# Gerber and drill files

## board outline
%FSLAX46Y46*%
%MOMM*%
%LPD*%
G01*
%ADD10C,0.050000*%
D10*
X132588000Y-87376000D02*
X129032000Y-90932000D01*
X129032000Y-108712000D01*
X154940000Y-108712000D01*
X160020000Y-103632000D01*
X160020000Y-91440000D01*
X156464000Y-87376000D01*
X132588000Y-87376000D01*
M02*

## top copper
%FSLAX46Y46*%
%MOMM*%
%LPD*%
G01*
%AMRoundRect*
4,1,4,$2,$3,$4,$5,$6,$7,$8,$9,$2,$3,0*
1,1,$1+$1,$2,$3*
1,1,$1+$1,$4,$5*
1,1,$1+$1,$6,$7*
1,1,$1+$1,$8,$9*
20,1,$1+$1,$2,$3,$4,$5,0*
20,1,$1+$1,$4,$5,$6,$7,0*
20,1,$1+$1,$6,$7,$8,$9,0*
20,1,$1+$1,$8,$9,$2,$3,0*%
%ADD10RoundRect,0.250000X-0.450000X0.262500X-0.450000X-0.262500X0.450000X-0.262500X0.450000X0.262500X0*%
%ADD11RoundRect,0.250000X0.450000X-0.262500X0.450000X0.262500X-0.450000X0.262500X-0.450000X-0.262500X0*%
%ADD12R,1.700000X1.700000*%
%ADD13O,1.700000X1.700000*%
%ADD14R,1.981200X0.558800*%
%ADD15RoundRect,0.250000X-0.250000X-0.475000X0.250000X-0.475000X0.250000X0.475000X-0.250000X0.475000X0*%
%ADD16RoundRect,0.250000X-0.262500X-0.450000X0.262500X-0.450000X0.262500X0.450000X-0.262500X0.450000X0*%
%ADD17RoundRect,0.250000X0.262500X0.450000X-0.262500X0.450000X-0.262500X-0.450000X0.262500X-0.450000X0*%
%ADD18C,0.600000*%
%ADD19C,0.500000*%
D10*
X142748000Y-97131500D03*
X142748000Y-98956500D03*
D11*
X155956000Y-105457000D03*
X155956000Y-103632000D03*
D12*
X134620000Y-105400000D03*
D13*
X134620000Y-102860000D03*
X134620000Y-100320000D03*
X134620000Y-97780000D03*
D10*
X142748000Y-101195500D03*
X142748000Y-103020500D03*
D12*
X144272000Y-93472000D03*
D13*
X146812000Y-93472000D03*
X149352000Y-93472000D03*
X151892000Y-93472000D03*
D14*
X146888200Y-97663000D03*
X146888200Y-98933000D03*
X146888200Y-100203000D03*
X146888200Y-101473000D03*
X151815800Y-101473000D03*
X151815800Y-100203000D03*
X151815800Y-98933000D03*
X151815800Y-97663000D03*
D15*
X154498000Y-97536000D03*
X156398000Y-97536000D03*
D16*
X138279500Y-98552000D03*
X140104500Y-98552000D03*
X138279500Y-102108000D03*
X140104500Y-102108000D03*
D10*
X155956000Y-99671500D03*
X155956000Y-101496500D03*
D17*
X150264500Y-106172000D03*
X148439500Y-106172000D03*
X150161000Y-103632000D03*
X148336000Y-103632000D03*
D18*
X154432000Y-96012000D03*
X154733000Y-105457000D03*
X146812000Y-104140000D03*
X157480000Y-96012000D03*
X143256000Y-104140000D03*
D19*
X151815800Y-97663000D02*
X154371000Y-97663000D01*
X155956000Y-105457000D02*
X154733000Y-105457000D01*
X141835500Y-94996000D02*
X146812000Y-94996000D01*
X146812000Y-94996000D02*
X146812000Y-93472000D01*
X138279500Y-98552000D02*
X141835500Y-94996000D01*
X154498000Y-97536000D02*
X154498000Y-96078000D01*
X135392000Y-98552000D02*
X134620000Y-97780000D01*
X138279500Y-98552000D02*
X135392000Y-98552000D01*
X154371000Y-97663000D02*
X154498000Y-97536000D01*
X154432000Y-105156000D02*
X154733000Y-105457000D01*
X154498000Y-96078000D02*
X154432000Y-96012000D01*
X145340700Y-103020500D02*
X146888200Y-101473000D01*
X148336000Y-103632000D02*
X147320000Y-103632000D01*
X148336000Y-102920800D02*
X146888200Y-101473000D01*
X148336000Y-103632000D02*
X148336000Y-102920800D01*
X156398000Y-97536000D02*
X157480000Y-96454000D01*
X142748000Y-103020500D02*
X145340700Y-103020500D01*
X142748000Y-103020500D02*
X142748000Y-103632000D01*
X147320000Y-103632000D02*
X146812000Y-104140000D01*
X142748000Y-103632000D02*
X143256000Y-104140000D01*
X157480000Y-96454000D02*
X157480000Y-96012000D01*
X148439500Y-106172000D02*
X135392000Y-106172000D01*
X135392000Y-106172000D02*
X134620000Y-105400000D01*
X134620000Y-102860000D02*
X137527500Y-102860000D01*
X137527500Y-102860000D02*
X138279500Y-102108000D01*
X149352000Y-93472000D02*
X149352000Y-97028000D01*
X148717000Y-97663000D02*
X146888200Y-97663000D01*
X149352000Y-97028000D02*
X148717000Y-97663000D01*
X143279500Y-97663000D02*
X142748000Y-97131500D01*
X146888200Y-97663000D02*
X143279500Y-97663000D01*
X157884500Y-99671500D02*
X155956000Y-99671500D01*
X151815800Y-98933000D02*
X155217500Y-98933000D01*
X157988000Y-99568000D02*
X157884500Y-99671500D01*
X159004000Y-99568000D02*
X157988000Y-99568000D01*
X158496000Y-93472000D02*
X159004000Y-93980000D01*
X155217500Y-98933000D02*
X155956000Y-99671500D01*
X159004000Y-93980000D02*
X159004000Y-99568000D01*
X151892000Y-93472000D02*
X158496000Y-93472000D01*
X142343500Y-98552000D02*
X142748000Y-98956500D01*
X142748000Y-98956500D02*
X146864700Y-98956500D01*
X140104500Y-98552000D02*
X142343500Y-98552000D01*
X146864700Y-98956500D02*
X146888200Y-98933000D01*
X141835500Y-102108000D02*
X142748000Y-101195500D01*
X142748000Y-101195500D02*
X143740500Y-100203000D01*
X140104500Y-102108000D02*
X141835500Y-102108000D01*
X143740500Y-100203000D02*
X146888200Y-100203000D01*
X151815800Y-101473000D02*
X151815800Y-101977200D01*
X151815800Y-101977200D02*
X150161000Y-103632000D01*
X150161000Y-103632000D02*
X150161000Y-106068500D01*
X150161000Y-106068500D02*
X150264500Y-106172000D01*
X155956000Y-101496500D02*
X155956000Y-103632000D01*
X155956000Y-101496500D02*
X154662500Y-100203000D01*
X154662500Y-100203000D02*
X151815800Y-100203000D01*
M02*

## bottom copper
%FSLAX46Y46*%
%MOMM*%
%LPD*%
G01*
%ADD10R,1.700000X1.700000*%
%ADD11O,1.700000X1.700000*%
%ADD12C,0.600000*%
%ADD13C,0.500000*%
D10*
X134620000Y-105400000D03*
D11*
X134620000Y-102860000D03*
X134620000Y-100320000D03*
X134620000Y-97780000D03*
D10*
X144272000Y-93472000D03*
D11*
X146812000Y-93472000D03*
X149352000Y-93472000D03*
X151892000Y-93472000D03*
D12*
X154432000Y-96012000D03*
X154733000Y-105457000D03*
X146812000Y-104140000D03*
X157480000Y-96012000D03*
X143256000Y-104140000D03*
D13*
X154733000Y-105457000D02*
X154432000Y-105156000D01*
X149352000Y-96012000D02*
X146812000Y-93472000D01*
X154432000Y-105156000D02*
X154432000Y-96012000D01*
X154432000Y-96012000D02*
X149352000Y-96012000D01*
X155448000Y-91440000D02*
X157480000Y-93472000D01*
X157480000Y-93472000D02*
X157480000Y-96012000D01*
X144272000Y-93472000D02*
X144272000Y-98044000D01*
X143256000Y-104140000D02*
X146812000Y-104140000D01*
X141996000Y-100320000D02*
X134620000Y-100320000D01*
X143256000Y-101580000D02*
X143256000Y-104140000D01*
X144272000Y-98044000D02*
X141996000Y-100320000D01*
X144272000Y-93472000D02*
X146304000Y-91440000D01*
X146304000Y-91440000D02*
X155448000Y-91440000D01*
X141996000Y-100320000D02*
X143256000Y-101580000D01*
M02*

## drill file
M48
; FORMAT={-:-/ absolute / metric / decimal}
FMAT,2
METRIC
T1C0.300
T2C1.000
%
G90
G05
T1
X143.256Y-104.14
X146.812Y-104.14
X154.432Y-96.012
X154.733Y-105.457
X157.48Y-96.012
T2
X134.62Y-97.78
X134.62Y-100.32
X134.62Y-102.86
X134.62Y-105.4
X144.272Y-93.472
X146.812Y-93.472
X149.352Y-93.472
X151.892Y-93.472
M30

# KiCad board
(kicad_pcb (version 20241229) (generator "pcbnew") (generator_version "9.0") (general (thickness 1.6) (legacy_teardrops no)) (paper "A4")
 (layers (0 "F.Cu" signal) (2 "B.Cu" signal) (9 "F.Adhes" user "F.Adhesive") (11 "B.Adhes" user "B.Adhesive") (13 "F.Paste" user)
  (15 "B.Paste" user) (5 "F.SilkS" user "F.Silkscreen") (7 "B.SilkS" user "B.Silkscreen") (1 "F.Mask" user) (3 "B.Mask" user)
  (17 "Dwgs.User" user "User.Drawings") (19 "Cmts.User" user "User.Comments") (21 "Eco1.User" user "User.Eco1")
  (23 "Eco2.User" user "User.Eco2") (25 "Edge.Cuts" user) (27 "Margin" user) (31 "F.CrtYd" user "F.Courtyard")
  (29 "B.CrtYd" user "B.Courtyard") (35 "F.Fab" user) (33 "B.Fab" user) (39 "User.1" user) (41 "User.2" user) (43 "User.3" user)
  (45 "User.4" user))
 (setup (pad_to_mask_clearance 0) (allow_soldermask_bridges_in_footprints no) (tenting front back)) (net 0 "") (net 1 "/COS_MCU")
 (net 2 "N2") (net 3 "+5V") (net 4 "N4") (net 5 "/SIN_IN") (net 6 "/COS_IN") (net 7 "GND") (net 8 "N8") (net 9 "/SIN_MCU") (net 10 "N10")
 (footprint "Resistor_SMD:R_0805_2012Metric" (layer "F.Cu") (at 142.748 98.044 -90)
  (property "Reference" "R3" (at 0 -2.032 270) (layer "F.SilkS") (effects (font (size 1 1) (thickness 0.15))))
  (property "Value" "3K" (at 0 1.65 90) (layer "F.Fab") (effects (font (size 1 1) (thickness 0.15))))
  (pad "1" smd roundrect (at -0.9125 0 270) (size 1.025 1.4) (layers "F.Cu" "F.Mask" "F.Paste") (roundrect_rratio 0.243902)
   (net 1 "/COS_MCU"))
  (pad "2" smd roundrect (at 0.9125 0 270) (size 1.025 1.4) (layers "F.Cu" "F.Mask" "F.Paste") (roundrect_rratio 0.243902) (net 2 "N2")))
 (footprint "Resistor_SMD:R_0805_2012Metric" (layer "F.Cu") (at 155.956 104.5445 90)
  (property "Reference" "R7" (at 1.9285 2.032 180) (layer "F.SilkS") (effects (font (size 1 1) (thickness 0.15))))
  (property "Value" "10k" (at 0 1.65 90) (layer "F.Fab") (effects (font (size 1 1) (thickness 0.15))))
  (pad "1" smd roundrect (at -0.9125 0 90) (size 1.025 1.4) (layers "F.Cu" "F.Mask" "F.Paste") (roundrect_rratio 0.243902) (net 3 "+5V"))
  (pad "2" smd roundrect (at 0.9125 0 90) (size 1.025 1.4) (layers "F.Cu" "F.Mask" "F.Paste") (roundrect_rratio 0.243902) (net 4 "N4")))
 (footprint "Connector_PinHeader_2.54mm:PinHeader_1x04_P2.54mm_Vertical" (layer "F.Cu") (at 134.62 105.4 180)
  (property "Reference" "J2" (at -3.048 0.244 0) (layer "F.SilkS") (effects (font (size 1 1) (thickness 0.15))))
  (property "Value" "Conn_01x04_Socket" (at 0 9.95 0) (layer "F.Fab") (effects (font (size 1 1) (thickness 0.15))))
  (pad "1" thru_hole rect (at 0 0 180) (size 1.7 1.7) (drill 1) (layers "*.Cu" "*.Mask") (remove_unused_layers no) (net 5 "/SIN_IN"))
  (pad "2" thru_hole oval (at 0 2.54 180) (size 1.7 1.7) (drill 1) (layers "*.Cu" "*.Mask") (remove_unused_layers no) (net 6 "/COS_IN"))
  (pad "3" thru_hole oval (at 0 5.08 180) (size 1.7 1.7) (drill 1) (layers "*.Cu" "*.Mask") (remove_unused_layers no) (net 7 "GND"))
  (pad "4" thru_hole oval (at 0 7.62 180) (size 1.7 1.7) (drill 1) (layers "*.Cu" "*.Mask") (remove_unused_layers no) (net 3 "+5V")))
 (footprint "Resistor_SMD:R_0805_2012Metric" (layer "F.Cu") (at 142.748 102.108 -90)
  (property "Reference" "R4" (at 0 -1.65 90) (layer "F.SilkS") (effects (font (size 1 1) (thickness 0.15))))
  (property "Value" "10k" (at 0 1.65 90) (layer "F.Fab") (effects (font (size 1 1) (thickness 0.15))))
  (pad "1" smd roundrect (at -0.9125 0 270) (size 1.025 1.4) (layers "F.Cu" "F.Mask" "F.Paste") (roundrect_rratio 0.243902) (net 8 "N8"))
  (pad "2" smd roundrect (at 0.9125 0 270) (size 1.025 1.4) (layers "F.Cu" "F.Mask" "F.Paste") (roundrect_rratio 0.243902) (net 7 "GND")))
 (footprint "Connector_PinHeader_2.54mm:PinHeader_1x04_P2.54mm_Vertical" (layer "F.Cu") (at 144.272 93.472 90)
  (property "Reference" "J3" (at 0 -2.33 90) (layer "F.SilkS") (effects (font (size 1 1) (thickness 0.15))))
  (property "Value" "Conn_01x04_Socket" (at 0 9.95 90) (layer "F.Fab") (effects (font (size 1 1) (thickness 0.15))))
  (pad "1" thru_hole rect (at 0 0 90) (size 1.7 1.7) (drill 1) (layers "*.Cu" "*.Mask") (remove_unused_layers no) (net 7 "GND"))
  (pad "2" thru_hole oval (at 0 2.54 90) (size 1.7 1.7) (drill 1) (layers "*.Cu" "*.Mask") (remove_unused_layers no) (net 3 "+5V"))
  (pad "3" thru_hole oval (at 0 5.08 90) (size 1.7 1.7) (drill 1) (layers "*.Cu" "*.Mask") (remove_unused_layers no) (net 1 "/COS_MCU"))
  (pad "4" thru_hole oval (at 0 7.62 90) (size 1.7 1.7) (drill 1) (layers "*.Cu" "*.Mask") (remove_unused_layers no) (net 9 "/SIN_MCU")))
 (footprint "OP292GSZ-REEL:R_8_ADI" (layer "F.Cu") (at 149.352 99.568)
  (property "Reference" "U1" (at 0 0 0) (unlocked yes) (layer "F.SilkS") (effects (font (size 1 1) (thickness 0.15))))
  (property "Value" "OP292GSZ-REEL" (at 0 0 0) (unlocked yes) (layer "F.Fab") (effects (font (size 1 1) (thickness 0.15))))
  (pad "1" smd rect (at -2.4638 -1.905) (size 1.9812 0.5588) (layers "F.Cu" "F.Mask" "F.Paste") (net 1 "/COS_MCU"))
  (pad "2" smd rect (at -2.4638 -0.635) (size 1.9812 0.5588) (layers "F.Cu" "F.Mask" "F.Paste") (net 2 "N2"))
  (pad "3" smd rect (at -2.4638 0.635) (size 1.9812 0.5588) (layers "F.Cu" "F.Mask" "F.Paste") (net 8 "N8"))
  (pad "4" smd rect (at -2.4638 1.905) (size 1.9812 0.5588) (layers "F.Cu" "F.Mask" "F.Paste") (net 7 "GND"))
  (pad "5" smd rect (at 2.4638 1.905) (size 1.9812 0.5588) (layers "F.Cu" "F.Mask" "F.Paste") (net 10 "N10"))
  (pad "6" smd rect (at 2.4638 0.635) (size 1.9812 0.5588) (layers "F.Cu" "F.Mask" "F.Paste") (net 4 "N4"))
  (pad "7" smd rect (at 2.4638 -0.635) (size 1.9812 0.5588) (layers "F.Cu" "F.Mask" "F.Paste") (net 9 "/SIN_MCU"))
  (pad "8" smd rect (at 2.4638 -1.905) (size 1.9812 0.5588) (layers "F.Cu" "F.Mask" "F.Paste") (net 3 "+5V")))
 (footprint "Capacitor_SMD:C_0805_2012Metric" (layer "F.Cu") (at 155.448 97.536)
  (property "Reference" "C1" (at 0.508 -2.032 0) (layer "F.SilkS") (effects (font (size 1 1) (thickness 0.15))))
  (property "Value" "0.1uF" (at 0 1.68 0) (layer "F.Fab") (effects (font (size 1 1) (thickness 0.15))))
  (pad "1" smd roundrect (at -0.95 0) (size 1 1.45) (layers "F.Cu" "F.Mask" "F.Paste") (roundrect_rratio 0.25) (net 3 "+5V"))
  (pad "2" smd roundrect (at 0.95 0) (size 1 1.45) (layers "F.Cu" "F.Mask" "F.Paste") (roundrect_rratio 0.25) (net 7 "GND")))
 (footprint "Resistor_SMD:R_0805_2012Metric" (layer "F.Cu") (at 139.192 98.552)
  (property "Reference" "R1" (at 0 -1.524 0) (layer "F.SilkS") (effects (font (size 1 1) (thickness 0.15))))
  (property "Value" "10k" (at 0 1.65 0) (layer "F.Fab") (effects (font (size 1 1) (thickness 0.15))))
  (pad "1" smd roundrect (at -0.9125 0) (size 1.025 1.4) (layers "F.Cu" "F.Mask" "F.Paste") (roundrect_rratio 0.243902) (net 3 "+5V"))
  (pad "2" smd roundrect (at 0.9125 0) (size 1.025 1.4) (layers "F.Cu" "F.Mask" "F.Paste") (roundrect_rratio 0.243902) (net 2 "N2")))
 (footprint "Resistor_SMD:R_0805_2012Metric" (layer "F.Cu") (at 139.192 102.108)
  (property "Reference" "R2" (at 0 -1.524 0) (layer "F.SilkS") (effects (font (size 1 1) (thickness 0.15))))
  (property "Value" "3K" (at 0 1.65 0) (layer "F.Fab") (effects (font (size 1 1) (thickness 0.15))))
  (pad "1" smd roundrect (at -0.9125 0) (size 1.025 1.4) (layers "F.Cu" "F.Mask" "F.Paste") (roundrect_rratio 0.243902) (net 6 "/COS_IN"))
  (pad "2" smd roundrect (at 0.9125 0) (size 1.025 1.4) (layers "F.Cu" "F.Mask" "F.Paste") (roundrect_rratio 0.243902) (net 8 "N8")))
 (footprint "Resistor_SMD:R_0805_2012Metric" (layer "F.Cu") (at 155.956 100.584 -90)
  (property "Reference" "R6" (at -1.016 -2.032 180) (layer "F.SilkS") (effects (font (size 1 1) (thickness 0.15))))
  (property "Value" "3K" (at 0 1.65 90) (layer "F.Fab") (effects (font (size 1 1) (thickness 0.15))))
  (pad "1" smd roundrect (at -0.9125 0 270) (size 1.025 1.4) (layers "F.Cu" "F.Mask" "F.Paste") (roundrect_rratio 0.243902)
   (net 9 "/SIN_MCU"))
  (pad "2" smd roundrect (at 0.9125 0 270) (size 1.025 1.4) (layers "F.Cu" "F.Mask" "F.Paste") (roundrect_rratio 0.243902) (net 4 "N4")))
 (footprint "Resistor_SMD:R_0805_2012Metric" (layer "F.Cu") (at 149.352 106.172 180)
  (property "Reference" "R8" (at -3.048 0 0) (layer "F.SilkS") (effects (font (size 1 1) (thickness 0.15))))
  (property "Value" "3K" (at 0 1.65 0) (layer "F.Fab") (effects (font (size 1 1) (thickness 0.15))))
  (pad "1" smd roundrect (at -0.9125 0 180) (size 1.025 1.4) (layers "F.Cu" "F.Mask" "F.Paste") (roundrect_rratio 0.243902) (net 10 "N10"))
  (pad "2" smd roundrect (at 0.9125 0 180) (size 1.025 1.4) (layers "F.Cu" "F.Mask" "F.Paste") (roundrect_rratio 0.243902) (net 5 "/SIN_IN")))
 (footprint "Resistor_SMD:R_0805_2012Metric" (layer "F.Cu") (at 149.2485 103.632 180)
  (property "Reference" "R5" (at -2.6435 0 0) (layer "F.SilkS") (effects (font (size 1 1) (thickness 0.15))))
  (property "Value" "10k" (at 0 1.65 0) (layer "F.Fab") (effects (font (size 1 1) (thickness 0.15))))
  (pad "1" smd roundrect (at -0.9125 0 180) (size 1.025 1.4) (layers "F.Cu" "F.Mask" "F.Paste") (roundrect_rratio 0.243902) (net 10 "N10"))
  (pad "2" smd roundrect (at 0.9125 0 180) (size 1.025 1.4) (layers "F.Cu" "F.Mask" "F.Paste") (roundrect_rratio 0.243902) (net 7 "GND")))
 (gr_poly
  (pts (xy 132.588 87.376) (xy 129.032 90.932) (xy 129.032 108.712) (xy 154.94 108.712) (xy 160.02 103.632) (xy 160.02 91.44)
   (xy 156.464 87.376))
  (stroke (width 0.05) (type solid)) (fill no) (layer "Edge.Cuts"))
 (segment (start 151.8158 97.663) (end 154.371 97.663) (width 0.5) (layer "F.Cu") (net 3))
 (segment (start 155.956 105.457) (end 154.733 105.457) (width 0.5) (layer "F.Cu") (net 3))
 (segment (start 141.8355 94.996) (end 146.812 94.996) (width 0.5) (layer "F.Cu") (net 3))
 (segment (start 146.812 94.996) (end 146.812 93.472) (width 0.5) (layer "F.Cu") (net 3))
 (segment (start 138.2795 98.552) (end 141.8355 94.996) (width 0.5) (layer "F.Cu") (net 3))
 (segment (start 154.498 97.536) (end 154.498 96.078) (width 0.5) (layer "F.Cu") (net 3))
 (segment (start 135.392 98.552) (end 134.62 97.78) (width 0.5) (layer "F.Cu") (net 3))
 (segment (start 138.2795 98.552) (end 135.392 98.552) (width 0.5) (layer "F.Cu") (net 3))
 (segment (start 154.371 97.663) (end 154.498 97.536) (width 0.5) (layer "F.Cu") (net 3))
 (segment (start 154.432 105.156) (end 154.733 105.457) (width 0.5) (layer "F.Cu") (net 3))
 (segment (start 154.498 96.078) (end 154.432 96.012) (width 0.5) (layer "F.Cu") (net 3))
 (via (at 154.432 96.012) (size 0.6) (drill 0.3) (layers "F.Cu" "B.Cu") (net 3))
 (via (at 154.733 105.457) (size 0.6) (drill 0.3) (layers "F.Cu" "B.Cu") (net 3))
 (segment (start 154.733 105.457) (end 154.432 105.156) (width 0.5) (layer "B.Cu") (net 3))
 (segment (start 149.352 96.012) (end 146.812 93.472) (width 0.5) (layer "B.Cu") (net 3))
 (segment (start 154.432 105.156) (end 154.432 96.012) (width 0.5) (layer "B.Cu") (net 3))
 (segment (start 154.432 96.012) (end 149.352 96.012) (width 0.5) (layer "B.Cu") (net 3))
 (segment (start 145.3407 103.0205) (end 146.8882 101.473) (width 0.5) (layer "F.Cu") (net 7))
 (segment (start 148.336 103.632) (end 147.32 103.632) (width 0.5) (layer "F.Cu") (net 7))
 (segment (start 148.336 102.9208) (end 146.8882 101.473) (width 0.5) (layer "F.Cu") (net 7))
 (segment (start 148.336 103.632) (end 148.336 102.9208) (width 0.5) (layer "F.Cu") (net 7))
 (segment (start 156.398 97.536) (end 157.48 96.454) (width 0.5) (layer "F.Cu") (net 7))
 (segment (start 142.748 103.0205) (end 145.3407 103.0205) (width 0.5) (layer "F.Cu") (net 7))
 (segment (start 142.748 103.0205) (end 142.748 103.632) (width 0.5) (layer "F.Cu") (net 7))
 (segment (start 147.32 103.632) (end 146.812 104.14) (width 0.5) (layer "F.Cu") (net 7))
 (segment (start 142.748 103.632) (end 143.256 104.14) (width 0.5) (layer "F.Cu") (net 7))
 (segment (start 157.48 96.454) (end 157.48 96.012) (width 0.5) (layer "F.Cu") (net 7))
 (via (at 146.812 104.14) (size 0.6) (drill 0.3) (layers "F.Cu" "B.Cu") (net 7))
 (via (at 157.48 96.012) (size 0.6) (drill 0.3) (layers "F.Cu" "B.Cu") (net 7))
 (via (at 143.256 104.14) (size 0.6) (drill 0.3) (layers "F.Cu" "B.Cu") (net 7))
 (segment (start 155.448 91.44) (end 157.48 93.472) (width 0.5) (layer "B.Cu") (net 7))
 (segment (start 157.48 93.472) (end 157.48 96.012) (width 0.5) (layer "B.Cu") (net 7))
 (segment (start 144.272 93.472) (end 144.272 98.044) (width 0.5) (layer "B.Cu") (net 7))
 (segment (start 143.256 104.14) (end 146.812 104.14) (width 0.5) (layer "B.Cu") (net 7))
 (segment (start 141.996 100.32) (end 134.62 100.32) (width 0.5) (layer "B.Cu") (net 7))
 (segment (start 143.256 101.58) (end 143.256 104.14) (width 0.5) (layer "B.Cu") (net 7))
 (segment (start 144.272 98.044) (end 141.996 100.32) (width 0.5) (layer "B.Cu") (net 7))
 (segment (start 144.272 93.472) (end 146.304 91.44) (width 0.5) (layer "B.Cu") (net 7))
 (segment (start 146.304 91.44) (end 155.448 91.44) (width 0.5) (layer "B.Cu") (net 7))
 (segment (start 141.996 100.32) (end 143.256 101.58) (width 0.5) (layer "B.Cu") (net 7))
 (segment (start 148.4395 106.172) (end 135.392 106.172) (width 0.5) (layer "F.Cu") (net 5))
 (segment (start 135.392 106.172) (end 134.62 105.4) (width 0.5) (layer "F.Cu") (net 5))
 (segment (start 134.62 102.86) (end 137.5275 102.86) (width 0.5) (layer "F.Cu") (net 6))
 (segment (start 137.5275 102.86) (end 138.2795 102.108) (width 0.5) (layer "F.Cu") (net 6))
 (segment (start 149.352 93.472) (end 149.352 97.028) (width 0.5) (layer "F.Cu") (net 1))
 (segment (start 148.717 97.663) (end 146.8882 97.663) (width 0.5) (layer "F.Cu") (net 1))
 (segment (start 149.352 97.028) (end 148.717 97.663) (width 0.5) (layer "F.Cu") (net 1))
 (segment (start 143.2795 97.663) (end 142.748 97.1315) (width 0.5) (layer "F.Cu") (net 1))
 (segment (start 146.8882 97.663) (end 143.2795 97.663) (width 0.5) (layer "F.Cu") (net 1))
 (segment (start 157.8845 99.6715) (end 155.956 99.6715) (width 0.5) (layer "F.Cu") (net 9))
 (segment (start 151.8158 98.933) (end 155.2175 98.933) (width 0.5) (layer "F.Cu") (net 9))
 (segment (start 157.988 99.568) (end 157.8845 99.6715) (width 0.5) (layer "F.Cu") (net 9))
 (segment (start 159.004 99.568) (end 157.988 99.568) (width 0.5) (layer "F.Cu") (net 9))
 (segment (start 158.496 93.472) (end 159.004 93.98) (width 0.5) (layer "F.Cu") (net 9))
 (segment (start 155.2175 98.933) (end 155.956 99.6715) (width 0.5) (layer "F.Cu") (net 9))
 (segment (start 159.004 93.98) (end 159.004 99.568) (width 0.5) (layer "F.Cu") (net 9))
 (segment (start 151.892 93.472) (end 158.496 93.472) (width 0.5) (layer "F.Cu") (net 9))
 (segment (start 142.3435 98.552) (end 142.748 98.9565) (width 0.5) (layer "F.Cu") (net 2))
 (segment (start 142.748 98.9565) (end 146.8647 98.9565) (width 0.5) (layer "F.Cu") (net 2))
 (segment (start 140.1045 98.552) (end 142.3435 98.552) (width 0.5) (layer "F.Cu") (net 2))
 (segment (start 146.8647 98.9565) (end 146.8882 98.933) (width 0.5) (layer "F.Cu") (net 2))
 (segment (start 141.8355 102.108) (end 142.748 101.1955) (width 0.5) (layer "F.Cu") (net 8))
 (segment (start 142.748 101.1955) (end 143.7405 100.203) (width 0.5) (layer "F.Cu") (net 8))
 (segment (start 140.1045 102.108) (end 141.8355 102.108) (width 0.5) (layer "F.Cu") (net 8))
 (segment (start 143.7405 100.203) (end 146.8882 100.203) (width 0.5) (layer "F.Cu") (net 8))
 (segment (start 151.8158 101.473) (end 151.8158 101.9772) (width 0.5) (layer "F.Cu") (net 10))
 (segment (start 151.8158 101.9772) (end 150.161 103.632) (width 0.5) (layer "F.Cu") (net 10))
 (segment (start 150.161 103.632) (end 150.161 106.0685) (width 0.5) (layer "F.Cu") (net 10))
 (segment (start 150.161 106.0685) (end 150.2645 106.172) (width 0.5) (layer "F.Cu") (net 10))
 (segment (start 155.956 101.4965) (end 155.956 103.632) (width 0.5) (layer "F.Cu") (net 4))
 (segment (start 155.956 101.4965) (end 154.6625 100.203) (width 0.5) (layer "F.Cu") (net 4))
 (segment (start 154.6625 100.203) (end 151.8158 100.203) (width 0.5) (layer "F.Cu") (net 4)))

